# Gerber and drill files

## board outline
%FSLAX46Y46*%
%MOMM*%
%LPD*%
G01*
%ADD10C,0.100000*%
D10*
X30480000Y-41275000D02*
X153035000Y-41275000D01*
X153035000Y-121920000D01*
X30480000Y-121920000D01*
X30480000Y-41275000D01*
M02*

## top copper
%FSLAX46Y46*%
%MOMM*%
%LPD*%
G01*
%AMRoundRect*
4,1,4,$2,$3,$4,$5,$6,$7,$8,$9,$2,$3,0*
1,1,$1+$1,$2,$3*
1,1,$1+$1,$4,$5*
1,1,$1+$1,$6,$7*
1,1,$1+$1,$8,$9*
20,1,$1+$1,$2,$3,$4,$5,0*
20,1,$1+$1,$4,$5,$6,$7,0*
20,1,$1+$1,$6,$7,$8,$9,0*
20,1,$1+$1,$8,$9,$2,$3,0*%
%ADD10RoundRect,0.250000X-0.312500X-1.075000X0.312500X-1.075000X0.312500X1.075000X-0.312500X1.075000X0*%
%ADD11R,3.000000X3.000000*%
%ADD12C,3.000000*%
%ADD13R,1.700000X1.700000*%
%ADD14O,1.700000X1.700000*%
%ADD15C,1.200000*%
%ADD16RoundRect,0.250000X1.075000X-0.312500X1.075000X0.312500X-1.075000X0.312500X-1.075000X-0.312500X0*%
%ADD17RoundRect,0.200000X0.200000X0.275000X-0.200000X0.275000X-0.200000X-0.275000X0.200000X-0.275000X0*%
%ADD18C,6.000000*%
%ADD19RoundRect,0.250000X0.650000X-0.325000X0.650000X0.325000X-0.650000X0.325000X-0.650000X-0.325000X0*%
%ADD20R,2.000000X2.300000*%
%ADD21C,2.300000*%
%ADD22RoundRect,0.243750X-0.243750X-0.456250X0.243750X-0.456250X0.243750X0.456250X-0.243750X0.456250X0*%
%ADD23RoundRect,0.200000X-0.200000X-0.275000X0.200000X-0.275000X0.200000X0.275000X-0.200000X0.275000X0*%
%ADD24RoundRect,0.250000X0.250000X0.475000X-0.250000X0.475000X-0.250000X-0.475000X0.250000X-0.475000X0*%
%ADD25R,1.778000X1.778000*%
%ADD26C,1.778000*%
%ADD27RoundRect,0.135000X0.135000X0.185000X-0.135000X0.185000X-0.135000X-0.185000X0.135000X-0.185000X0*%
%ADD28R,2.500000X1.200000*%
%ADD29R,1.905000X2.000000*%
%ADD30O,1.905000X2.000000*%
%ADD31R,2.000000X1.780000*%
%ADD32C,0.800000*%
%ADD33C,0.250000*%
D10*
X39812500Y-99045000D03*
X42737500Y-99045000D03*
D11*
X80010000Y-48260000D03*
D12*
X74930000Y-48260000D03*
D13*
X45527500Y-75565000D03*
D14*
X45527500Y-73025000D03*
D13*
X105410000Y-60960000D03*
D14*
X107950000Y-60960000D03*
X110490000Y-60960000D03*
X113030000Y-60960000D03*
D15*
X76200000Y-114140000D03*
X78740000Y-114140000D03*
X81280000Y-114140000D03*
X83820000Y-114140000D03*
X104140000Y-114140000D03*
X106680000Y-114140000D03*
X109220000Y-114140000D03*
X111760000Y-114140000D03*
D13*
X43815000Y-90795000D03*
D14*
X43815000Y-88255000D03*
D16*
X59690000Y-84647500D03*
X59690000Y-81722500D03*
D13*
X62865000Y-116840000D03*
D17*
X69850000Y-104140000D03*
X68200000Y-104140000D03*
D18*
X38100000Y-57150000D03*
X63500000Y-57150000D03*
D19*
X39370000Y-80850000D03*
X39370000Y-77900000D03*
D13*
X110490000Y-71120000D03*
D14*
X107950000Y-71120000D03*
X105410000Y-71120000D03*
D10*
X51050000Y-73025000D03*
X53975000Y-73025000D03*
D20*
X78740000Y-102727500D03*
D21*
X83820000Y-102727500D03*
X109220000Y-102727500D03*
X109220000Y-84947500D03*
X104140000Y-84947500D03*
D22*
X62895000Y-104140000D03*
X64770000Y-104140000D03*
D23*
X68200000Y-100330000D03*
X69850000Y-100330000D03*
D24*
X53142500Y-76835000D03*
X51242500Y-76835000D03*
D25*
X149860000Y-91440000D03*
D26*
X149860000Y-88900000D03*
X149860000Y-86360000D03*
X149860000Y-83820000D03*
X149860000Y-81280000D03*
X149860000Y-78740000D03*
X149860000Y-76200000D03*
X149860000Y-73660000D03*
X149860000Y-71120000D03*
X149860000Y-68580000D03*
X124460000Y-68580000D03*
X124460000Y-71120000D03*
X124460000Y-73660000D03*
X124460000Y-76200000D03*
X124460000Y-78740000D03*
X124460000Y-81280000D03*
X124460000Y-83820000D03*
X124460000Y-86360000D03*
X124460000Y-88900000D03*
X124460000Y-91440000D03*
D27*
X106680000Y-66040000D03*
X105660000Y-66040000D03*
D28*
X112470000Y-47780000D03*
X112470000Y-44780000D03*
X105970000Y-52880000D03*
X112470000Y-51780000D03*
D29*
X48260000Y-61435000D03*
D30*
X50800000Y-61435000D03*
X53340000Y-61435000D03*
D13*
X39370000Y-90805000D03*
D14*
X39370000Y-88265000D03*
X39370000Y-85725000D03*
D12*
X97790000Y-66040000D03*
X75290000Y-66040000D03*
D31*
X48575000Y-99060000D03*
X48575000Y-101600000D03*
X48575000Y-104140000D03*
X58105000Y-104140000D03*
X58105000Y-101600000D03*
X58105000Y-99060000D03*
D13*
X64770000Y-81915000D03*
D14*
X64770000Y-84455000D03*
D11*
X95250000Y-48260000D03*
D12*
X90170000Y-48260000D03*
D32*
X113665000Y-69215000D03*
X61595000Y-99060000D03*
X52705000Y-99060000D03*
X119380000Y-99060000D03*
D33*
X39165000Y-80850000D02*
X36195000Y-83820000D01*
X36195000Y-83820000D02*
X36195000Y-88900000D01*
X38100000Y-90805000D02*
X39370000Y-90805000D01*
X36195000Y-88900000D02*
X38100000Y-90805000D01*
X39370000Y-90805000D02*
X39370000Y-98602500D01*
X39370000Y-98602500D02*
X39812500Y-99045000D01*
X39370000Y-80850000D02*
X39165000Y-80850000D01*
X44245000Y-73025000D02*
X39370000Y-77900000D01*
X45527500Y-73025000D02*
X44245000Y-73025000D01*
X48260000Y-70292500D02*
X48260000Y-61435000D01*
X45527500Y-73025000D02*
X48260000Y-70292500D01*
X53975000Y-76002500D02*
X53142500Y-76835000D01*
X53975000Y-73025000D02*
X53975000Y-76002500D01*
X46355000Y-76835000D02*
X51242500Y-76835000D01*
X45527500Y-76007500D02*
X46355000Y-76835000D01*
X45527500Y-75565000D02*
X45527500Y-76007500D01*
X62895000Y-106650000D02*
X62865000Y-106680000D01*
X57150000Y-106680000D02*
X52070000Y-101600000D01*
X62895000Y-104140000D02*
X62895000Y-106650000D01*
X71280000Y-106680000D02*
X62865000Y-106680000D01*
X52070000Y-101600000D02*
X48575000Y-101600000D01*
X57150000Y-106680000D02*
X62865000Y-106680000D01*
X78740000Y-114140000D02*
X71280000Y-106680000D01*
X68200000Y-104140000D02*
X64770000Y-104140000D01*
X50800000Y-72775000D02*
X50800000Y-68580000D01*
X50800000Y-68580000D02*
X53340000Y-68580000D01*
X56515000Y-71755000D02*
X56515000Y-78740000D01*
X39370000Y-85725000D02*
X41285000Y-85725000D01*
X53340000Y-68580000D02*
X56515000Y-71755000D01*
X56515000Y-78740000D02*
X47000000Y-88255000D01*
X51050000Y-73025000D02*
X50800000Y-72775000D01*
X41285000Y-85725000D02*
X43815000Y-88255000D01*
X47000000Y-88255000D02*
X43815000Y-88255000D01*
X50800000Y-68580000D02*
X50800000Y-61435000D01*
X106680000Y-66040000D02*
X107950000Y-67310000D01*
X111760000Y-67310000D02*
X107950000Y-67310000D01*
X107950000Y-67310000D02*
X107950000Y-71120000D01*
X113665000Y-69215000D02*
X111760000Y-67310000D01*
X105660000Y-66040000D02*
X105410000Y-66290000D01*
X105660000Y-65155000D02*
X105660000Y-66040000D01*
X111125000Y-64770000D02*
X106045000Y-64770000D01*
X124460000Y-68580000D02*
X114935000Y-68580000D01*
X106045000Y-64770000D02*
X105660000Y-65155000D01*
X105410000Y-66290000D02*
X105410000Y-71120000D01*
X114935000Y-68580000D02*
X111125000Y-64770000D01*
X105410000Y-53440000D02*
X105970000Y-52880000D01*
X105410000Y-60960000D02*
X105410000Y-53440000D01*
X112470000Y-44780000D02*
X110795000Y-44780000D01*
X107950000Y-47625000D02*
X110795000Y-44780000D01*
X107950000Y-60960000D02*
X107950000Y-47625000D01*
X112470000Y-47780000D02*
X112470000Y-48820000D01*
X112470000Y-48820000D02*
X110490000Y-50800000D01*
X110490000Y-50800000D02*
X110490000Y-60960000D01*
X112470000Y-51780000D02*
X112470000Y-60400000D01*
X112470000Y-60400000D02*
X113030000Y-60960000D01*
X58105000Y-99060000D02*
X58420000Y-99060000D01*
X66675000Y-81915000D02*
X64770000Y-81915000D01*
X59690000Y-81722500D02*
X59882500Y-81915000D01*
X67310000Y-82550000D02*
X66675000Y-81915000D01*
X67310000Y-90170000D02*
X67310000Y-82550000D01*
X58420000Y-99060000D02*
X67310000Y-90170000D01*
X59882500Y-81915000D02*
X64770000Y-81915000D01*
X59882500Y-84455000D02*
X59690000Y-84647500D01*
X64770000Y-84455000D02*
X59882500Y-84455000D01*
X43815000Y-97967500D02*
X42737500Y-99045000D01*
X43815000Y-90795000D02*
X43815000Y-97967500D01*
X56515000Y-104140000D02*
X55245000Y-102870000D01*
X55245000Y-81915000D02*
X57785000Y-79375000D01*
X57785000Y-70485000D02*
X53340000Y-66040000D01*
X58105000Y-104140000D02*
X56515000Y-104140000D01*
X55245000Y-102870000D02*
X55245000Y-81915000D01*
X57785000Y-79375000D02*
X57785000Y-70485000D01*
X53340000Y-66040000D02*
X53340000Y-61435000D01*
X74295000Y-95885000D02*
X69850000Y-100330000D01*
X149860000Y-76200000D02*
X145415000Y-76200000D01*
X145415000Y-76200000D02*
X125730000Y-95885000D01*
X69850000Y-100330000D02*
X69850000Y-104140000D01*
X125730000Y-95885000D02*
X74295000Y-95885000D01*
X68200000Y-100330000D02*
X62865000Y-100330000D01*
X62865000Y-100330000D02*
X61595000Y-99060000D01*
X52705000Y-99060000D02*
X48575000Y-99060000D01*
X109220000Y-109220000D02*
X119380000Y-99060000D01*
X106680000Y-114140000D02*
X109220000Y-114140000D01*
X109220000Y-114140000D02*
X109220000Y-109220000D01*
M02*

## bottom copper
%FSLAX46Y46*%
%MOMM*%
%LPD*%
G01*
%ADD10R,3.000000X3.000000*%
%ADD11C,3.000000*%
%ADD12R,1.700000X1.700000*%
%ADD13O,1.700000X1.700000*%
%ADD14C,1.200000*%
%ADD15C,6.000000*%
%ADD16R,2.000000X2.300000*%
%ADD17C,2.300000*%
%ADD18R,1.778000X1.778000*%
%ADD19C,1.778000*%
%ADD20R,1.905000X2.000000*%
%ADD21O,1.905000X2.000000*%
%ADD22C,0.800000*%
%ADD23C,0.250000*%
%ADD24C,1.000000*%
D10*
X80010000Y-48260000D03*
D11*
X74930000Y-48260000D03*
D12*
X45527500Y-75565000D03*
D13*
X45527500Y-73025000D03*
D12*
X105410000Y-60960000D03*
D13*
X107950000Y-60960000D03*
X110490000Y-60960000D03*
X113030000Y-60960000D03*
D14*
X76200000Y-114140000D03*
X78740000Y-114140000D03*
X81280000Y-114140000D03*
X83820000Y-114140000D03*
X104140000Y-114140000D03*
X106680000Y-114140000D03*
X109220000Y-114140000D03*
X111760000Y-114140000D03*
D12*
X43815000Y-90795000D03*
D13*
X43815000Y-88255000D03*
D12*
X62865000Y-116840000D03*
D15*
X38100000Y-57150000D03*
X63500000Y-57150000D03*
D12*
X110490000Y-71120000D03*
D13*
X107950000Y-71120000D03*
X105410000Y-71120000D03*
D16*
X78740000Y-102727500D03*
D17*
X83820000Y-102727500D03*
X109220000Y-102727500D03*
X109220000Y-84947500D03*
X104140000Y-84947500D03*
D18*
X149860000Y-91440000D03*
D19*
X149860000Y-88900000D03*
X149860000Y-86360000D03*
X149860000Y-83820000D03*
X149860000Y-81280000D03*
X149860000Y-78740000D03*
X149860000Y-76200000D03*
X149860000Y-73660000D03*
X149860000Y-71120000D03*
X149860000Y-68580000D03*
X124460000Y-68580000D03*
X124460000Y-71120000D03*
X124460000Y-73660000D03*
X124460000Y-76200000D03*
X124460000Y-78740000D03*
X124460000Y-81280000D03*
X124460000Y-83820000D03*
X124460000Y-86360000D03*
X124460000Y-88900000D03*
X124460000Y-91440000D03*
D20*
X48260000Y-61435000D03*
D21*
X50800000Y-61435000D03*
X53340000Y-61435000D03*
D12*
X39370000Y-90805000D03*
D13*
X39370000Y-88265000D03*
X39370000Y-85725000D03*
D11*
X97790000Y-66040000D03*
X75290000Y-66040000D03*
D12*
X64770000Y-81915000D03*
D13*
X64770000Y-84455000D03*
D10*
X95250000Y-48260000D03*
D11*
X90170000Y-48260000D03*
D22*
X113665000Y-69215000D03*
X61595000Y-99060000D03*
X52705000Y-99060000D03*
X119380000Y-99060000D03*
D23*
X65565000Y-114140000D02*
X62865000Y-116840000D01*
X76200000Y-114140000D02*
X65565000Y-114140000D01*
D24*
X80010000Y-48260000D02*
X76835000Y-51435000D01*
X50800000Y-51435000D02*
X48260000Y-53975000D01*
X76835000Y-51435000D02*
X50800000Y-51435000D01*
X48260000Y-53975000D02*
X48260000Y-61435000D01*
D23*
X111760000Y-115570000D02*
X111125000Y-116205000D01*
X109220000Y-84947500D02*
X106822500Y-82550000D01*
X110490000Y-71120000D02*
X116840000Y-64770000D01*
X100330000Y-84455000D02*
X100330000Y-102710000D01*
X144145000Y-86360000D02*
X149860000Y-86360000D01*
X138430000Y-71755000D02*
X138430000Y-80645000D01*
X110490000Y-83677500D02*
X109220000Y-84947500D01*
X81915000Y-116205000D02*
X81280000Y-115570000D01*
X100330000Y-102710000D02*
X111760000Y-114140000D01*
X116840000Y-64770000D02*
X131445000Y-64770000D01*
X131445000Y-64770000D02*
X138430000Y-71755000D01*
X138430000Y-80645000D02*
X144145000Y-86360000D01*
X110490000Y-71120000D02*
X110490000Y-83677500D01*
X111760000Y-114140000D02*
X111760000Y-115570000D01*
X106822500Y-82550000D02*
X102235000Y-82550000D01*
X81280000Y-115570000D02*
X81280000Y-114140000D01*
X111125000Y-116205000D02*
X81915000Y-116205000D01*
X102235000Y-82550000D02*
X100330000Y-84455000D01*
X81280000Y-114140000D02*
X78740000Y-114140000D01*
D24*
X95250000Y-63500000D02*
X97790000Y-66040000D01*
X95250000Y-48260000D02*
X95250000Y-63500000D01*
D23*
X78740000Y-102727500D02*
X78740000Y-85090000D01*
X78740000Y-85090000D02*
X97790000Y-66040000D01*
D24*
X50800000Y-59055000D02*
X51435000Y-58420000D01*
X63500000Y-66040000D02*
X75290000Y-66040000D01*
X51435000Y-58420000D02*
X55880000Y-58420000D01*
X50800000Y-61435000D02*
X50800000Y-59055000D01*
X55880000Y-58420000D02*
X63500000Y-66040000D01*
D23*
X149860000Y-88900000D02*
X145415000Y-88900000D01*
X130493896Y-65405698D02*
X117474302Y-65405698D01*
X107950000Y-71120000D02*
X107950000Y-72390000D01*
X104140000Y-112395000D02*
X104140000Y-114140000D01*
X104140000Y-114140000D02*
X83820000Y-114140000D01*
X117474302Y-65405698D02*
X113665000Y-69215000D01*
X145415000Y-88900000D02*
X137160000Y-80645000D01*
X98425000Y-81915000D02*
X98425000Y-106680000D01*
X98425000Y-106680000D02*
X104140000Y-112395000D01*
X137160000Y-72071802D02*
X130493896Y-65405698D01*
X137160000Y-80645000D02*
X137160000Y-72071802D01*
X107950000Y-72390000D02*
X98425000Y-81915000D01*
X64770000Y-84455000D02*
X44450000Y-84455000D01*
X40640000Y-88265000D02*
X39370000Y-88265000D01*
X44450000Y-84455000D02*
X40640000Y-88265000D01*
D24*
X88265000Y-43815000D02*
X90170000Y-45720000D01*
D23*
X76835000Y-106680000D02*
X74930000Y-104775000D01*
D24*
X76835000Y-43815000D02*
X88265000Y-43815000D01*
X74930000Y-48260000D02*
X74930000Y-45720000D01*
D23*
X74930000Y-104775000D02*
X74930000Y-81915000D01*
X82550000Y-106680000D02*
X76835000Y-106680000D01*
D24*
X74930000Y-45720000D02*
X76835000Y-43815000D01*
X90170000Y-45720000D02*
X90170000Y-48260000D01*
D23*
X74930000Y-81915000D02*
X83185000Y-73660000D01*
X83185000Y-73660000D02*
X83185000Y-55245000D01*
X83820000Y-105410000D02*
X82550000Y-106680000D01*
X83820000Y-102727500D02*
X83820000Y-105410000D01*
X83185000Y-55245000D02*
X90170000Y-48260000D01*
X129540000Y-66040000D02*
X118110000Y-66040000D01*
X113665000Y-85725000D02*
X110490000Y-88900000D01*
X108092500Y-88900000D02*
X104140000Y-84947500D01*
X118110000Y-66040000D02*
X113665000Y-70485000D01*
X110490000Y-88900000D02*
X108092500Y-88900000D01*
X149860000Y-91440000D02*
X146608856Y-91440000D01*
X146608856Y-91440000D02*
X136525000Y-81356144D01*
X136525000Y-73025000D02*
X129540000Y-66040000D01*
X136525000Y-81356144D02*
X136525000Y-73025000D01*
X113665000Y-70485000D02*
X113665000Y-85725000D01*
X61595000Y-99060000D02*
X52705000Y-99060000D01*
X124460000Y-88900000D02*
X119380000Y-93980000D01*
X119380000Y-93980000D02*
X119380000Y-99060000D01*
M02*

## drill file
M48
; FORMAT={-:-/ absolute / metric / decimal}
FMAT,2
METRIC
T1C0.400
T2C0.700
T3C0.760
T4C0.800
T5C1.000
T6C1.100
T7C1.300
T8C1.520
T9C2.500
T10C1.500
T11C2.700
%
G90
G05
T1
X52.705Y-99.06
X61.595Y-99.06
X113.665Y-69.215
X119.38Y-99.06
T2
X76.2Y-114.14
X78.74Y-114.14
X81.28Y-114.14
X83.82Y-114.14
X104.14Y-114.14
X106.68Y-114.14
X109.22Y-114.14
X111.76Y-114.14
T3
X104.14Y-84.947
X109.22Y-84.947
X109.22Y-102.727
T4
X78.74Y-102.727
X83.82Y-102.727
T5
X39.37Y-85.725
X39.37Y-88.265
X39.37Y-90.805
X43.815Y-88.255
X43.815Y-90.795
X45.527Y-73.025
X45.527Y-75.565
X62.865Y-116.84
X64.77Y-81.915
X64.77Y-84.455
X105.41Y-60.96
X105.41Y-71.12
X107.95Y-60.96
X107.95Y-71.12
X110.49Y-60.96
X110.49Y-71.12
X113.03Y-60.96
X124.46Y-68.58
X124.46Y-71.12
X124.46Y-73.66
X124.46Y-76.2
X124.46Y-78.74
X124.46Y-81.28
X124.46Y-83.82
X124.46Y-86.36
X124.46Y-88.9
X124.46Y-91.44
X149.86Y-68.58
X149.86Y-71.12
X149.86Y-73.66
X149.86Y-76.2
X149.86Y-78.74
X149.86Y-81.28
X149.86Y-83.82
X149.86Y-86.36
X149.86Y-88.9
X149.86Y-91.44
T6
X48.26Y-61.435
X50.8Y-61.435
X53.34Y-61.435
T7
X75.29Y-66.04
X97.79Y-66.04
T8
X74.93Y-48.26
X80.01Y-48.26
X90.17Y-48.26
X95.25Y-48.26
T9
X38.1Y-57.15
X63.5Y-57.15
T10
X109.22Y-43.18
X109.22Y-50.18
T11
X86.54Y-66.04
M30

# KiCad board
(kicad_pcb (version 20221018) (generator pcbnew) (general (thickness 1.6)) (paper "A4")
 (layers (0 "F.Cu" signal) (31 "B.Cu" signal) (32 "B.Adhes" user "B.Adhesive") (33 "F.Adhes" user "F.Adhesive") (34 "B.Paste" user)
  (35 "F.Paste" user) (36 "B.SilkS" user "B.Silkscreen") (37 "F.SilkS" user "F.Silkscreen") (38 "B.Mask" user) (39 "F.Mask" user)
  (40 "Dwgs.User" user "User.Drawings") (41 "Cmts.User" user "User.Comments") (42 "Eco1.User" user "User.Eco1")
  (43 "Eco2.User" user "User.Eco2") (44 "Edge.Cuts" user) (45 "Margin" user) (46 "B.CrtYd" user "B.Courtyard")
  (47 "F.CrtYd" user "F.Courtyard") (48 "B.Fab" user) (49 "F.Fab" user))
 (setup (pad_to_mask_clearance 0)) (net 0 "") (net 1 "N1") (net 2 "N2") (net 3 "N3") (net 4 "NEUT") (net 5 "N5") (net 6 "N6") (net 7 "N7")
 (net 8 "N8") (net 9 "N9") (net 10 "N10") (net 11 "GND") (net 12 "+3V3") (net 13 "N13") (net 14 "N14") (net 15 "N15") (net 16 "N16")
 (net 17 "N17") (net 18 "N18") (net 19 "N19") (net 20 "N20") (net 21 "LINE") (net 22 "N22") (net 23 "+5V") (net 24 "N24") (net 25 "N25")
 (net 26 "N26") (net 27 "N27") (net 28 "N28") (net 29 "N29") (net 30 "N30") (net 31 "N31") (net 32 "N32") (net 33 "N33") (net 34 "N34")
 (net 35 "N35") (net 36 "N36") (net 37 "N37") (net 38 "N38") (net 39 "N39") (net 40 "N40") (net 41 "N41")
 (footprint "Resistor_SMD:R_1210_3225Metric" (layer "F.Cu") (at 41.275 99.045)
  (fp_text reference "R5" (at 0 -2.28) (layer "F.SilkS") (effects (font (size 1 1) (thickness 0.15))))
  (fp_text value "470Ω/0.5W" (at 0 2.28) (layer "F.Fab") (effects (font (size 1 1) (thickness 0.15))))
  (pad "1" smd roundrect (at -1.4625 0) (size 1.125 2.65) (layers "F.Cu" "F.Paste" "F.Mask") (roundrect_rratio 0.222222) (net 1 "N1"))
  (pad "2" smd roundrect (at 1.4625 0) (size 1.125 2.65) (layers "F.Cu" "F.Paste" "F.Mask") (roundrect_rratio 0.222222) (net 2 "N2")))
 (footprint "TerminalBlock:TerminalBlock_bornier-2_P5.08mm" (layer "F.Cu") (at 80.01 48.26 180)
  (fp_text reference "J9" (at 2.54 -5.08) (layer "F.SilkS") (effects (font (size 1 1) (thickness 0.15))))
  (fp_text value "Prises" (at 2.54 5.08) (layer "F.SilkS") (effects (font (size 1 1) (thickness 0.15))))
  (pad "1" thru_hole rect (at 0 0 180) (size 3 3) (drill 1.52) (layers "*.Cu" "*.Mask") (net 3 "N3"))
  (pad "2" thru_hole circle (at 5.08 0 180) (size 3 3) (drill 1.52) (layers "*.Cu" "*.Mask") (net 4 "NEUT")))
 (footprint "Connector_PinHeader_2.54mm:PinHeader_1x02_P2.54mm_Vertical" (layer "F.Cu") (at 45.5275 75.565 180)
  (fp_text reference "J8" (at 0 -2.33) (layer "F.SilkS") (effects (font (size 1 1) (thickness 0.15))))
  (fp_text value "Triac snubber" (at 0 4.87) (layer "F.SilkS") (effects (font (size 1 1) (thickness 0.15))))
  (pad "1" thru_hole rect (at 0 0 180) (size 1.7 1.7) (drill 1) (layers "*.Cu" "*.Mask") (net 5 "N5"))
  (pad "2" thru_hole oval (at 0 2.54 180) (size 1.7 1.7) (drill 1) (layers "*.Cu" "*.Mask") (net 3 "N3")))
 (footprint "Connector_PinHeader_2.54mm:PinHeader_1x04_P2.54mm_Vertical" (layer "F.Cu") (at 105.41 60.96 90)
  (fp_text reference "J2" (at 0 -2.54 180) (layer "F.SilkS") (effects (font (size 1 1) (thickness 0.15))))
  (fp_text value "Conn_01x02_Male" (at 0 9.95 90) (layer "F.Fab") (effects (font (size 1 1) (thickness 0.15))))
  (pad "1" thru_hole rect (at 0 0 90) (size 1.7 1.7) (drill 1) (layers "*.Cu" "*.Mask") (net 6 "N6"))
  (pad "2" thru_hole oval (at 0 2.54 90) (size 1.7 1.7) (drill 1) (layers "*.Cu" "*.Mask") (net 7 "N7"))
  (pad "3" thru_hole oval (at 0 5.08 90) (size 1.7 1.7) (drill 1) (layers "*.Cu" "*.Mask") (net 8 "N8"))
  (pad "4" thru_hole oval (at 0 7.62 90) (size 1.7 1.7) (drill 1) (layers "*.Cu" "*.Mask") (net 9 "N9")))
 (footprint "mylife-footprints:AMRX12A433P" (layer "F.Cu") (at 93.98 116.84)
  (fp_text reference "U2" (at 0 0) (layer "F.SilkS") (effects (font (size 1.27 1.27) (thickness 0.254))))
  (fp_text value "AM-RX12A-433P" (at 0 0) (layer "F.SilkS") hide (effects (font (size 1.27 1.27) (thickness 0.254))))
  (pad "1" thru_hole circle (at -17.78 -2.7) (size 1.2 1.2) (drill 0.7) (layers "*.Cu" "*.Mask") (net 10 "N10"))
  (pad "2" thru_hole circle (at -15.24 -2.7) (size 1.2 1.2) (drill 0.7) (layers "*.Cu" "*.Mask") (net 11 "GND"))
  (pad "3" thru_hole circle (at -12.7 -2.7) (size 1.2 1.2) (drill 0.7) (layers "*.Cu" "*.Mask") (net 11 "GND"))
  (pad "4" thru_hole circle (at -10.16 -2.7) (size 1.2 1.2) (drill 0.7) (layers "*.Cu" "*.Mask") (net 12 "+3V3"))
  (pad "5" thru_hole circle (at 10.16 -2.7) (size 1.2 1.2) (drill 0.7) (layers "*.Cu" "*.Mask") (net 12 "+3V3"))
  (pad "6" thru_hole circle (at 12.7 -2.7) (size 1.2 1.2) (drill 0.7) (layers "*.Cu" "*.Mask") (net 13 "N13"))
  (pad "7" thru_hole circle (at 15.24 -2.7) (size 1.2 1.2) (drill 0.7) (layers "*.Cu" "*.Mask") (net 13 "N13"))
  (pad "8" thru_hole circle (at 17.78 -2.7) (size 1.2 1.2) (drill 0.7) (layers "*.Cu" "*.Mask") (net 11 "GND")))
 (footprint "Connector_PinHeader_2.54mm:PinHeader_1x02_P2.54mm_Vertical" (layer "F.Cu") (at 43.815 90.795 180)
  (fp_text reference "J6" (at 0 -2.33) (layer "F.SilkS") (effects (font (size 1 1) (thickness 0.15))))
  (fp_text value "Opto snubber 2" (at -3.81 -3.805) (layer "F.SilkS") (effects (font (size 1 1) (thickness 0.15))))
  (pad "1" thru_hole rect (at 0 0 180) (size 1.7 1.7) (drill 1) (layers "*.Cu" "*.Mask") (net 2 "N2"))
  (pad "2" thru_hole oval (at 0 2.54 180) (size 1.7 1.7) (drill 1) (layers "*.Cu" "*.Mask") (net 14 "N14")))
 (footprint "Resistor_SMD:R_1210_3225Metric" (layer "F.Cu") (at 59.69 83.185 90)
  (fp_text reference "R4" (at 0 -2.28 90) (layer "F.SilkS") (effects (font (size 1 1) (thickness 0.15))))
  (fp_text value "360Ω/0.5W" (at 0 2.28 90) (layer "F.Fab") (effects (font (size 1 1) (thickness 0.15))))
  (pad "1" smd roundrect (at -1.4625 0 90) (size 1.125 2.65) (layers "F.Cu" "F.Paste" "F.Mask") (roundrect_rratio 0.222222) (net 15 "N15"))
  (pad "2" smd roundrect (at 1.4625 0 90) (size 1.125 2.65) (layers "F.Cu" "F.Paste" "F.Mask") (roundrect_rratio 0.222222) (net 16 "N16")))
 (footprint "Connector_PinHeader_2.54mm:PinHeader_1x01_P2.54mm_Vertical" (layer "F.Cu") (at 62.865 116.84)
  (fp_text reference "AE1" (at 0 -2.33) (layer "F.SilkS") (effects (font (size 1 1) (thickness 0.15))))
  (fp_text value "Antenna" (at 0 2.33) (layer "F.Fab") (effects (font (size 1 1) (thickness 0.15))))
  (pad "1" thru_hole rect (at 0 0) (size 1.7 1.7) (drill 1) (layers "*.Cu" "*.Mask") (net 10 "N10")))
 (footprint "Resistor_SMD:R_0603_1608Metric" (layer "F.Cu") (at 69.025 104.14 180)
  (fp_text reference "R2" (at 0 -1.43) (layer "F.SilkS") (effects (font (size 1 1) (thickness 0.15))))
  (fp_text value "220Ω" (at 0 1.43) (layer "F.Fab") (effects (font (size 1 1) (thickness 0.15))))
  (pad "1" smd roundrect (at -0.825 0 180) (size 0.8 0.95) (layers "F.Cu" "F.Paste" "F.Mask") (roundrect_rratio 0.25) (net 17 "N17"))
  (pad "2" smd roundrect (at 0.825 0 180) (size 0.8 0.95) (layers "F.Cu" "F.Paste" "F.Mask") (roundrect_rratio 0.25) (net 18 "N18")))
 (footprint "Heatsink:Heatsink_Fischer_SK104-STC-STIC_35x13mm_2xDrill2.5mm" (layer "F.Cu") (at 50.8 57.15)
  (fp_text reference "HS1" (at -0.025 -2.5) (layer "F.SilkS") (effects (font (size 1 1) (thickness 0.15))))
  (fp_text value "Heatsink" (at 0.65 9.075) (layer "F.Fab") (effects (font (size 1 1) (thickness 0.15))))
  (pad "1" thru_hole circle (at -12.7 0 180) (size 6 6) (drill 2.5) (layers "*.Cu" "*.Mask"))
  (pad "1" thru_hole circle (at 12.7 0) (size 6 6) (drill 2.5) (layers "*.Cu" "*.Mask")))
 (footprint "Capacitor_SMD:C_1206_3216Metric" (layer "F.Cu") (at 39.37 79.375 90)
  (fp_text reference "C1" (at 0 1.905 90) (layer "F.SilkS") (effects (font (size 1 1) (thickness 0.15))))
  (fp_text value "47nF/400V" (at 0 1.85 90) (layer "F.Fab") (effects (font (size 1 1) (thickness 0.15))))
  (pad "1" smd roundrect (at -1.475 0 90) (size 1.15 1.8) (layers "F.Cu" "F.Paste" "F.Mask") (roundrect_rratio 0.217391) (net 1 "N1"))
  (pad "2" smd roundrect (at 1.475 0 90) (size 1.15 1.8) (layers "F.Cu" "F.Paste" "F.Mask") (roundrect_rratio 0.217391) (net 3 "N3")))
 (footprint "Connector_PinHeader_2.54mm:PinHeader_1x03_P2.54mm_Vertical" (layer "F.Cu") (at 110.49 71.12 -90)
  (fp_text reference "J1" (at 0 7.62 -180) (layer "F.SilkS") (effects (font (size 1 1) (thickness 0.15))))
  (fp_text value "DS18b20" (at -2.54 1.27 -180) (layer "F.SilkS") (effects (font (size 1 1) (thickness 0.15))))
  (pad "1" thru_hole rect (at 0 0 270) (size 1.7 1.7) (drill 1) (layers "*.Cu" "*.Mask") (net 11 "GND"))
  (pad "2" thru_hole oval (at 0 2.54 270) (size 1.7 1.7) (drill 1) (layers "*.Cu" "*.Mask") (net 12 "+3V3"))
  (pad "3" thru_hole oval (at 0 5.08 270) (size 1.7 1.7) (drill 1) (layers "*.Cu" "*.Mask") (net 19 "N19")))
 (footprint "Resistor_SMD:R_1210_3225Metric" (layer "F.Cu") (at 52.5125 73.025)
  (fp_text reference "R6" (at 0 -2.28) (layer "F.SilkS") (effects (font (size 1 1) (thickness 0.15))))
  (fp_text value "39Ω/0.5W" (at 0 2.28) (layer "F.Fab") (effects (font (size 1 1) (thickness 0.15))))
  (pad "1" smd roundrect (at -1.4625 0) (size 1.125 2.65) (layers "F.Cu" "F.Paste" "F.Mask") (roundrect_rratio 0.222222) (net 14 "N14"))
  (pad "2" smd roundrect (at 1.4625 0) (size 1.125 2.65) (layers "F.Cu" "F.Paste" "F.Mask") (roundrect_rratio 0.222222) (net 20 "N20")))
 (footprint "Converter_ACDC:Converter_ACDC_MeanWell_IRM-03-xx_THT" (layer "F.Cu") (at 78.74 102.7275 90)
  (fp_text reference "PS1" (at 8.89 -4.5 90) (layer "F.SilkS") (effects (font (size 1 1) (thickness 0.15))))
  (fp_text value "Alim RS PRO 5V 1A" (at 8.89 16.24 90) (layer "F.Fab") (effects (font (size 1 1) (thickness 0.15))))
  (pad "1" thru_hole rect (at 0 0 90) (size 2.3 2) (drill 0.8) (layers "*.Cu" "*.Mask") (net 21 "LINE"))
  (pad "3" thru_hole circle (at 0 5.08 90) (size 2.3 2.3) (drill 0.8) (layers "*.Cu" "*.Mask") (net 4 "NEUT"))
  (pad "5" thru_hole circle (at 0 30.48 90) (size 2.3 2.3) (drill 0.76) (layers "*.Cu" "*.Mask") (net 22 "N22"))
  (pad "14" thru_hole circle (at 17.78 30.48 90) (size 2.3 2.3) (drill 0.76) (layers "*.Cu" "*.Mask") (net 11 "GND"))
  (pad "16" thru_hole circle (at 17.78 25.4 90) (size 2.3 2.3) (drill 0.76) (layers "*.Cu" "*.Mask") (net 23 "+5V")))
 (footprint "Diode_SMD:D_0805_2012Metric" (layer "F.Cu") (at 63.8325 104.14)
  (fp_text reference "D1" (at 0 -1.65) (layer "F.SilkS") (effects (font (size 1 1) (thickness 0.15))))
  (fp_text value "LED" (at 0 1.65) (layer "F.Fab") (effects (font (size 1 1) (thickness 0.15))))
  (pad "1" smd roundrect (at -0.9375 0) (size 0.975 1.4) (layers "F.Cu" "F.Paste" "F.Mask") (roundrect_rratio 0.25) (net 11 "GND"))
  (pad "2" smd roundrect (at 0.9375 0) (size 0.975 1.4) (layers "F.Cu" "F.Paste" "F.Mask") (roundrect_rratio 0.25) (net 18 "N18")))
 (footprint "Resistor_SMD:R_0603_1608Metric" (layer "F.Cu") (at 69.025 100.33)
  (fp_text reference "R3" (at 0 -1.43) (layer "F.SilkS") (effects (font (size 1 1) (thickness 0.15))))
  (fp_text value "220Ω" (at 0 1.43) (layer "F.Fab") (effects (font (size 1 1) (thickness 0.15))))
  (pad "1" smd roundrect (at -0.825 0) (size 0.8 0.95) (layers "F.Cu" "F.Paste" "F.Mask") (roundrect_rratio 0.25) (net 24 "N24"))
  (pad "2" smd roundrect (at 0.825 0) (size 0.8 0.95) (layers "F.Cu" "F.Paste" "F.Mask") (roundrect_rratio 0.25) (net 17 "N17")))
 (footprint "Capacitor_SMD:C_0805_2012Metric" (layer "F.Cu") (at 52.1925 76.835 180)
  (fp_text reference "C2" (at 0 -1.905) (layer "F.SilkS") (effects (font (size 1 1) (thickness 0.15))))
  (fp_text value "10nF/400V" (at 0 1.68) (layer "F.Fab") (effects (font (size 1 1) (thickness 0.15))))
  (pad "1" smd roundrect (at -0.95 0 180) (size 1 1.45) (layers "F.Cu" "F.Paste" "F.Mask") (roundrect_rratio 0.25) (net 20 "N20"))
  (pad "2" smd roundrect (at 0.95 0 180) (size 1 1.45) (layers "F.Cu" "F.Paste" "F.Mask") (roundrect_rratio 0.25) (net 5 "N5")))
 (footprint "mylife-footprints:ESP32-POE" (layer "F.Cu") (at 137.12 81.41 180)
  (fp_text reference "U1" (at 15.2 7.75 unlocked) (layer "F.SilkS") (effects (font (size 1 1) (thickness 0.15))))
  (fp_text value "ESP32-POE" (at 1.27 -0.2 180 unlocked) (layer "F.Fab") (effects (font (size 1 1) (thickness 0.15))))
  (pad "1" thru_hole rect (at -12.74 -10.03 90) (size 1.778 1.778) (drill 1) (layers "*.Cu" "*.Mask") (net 23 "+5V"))
  (pad "2" thru_hole circle (at -12.74 -7.49 90) (size 1.778 1.778) (drill 1) (layers "*.Cu" "*.Mask") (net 12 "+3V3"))
  (pad "3" thru_hole circle (at -12.74 -4.95 90) (size 1.778 1.778) (drill 1) (layers "*.Cu" "*.Mask") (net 11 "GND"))
  (pad "4" thru_hole circle (at -12.74 -2.41 90) (size 1.778 1.778) (drill 1) (layers "*.Cu" "*.Mask") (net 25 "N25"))
  (pad "5" thru_hole circle (at -12.74 0.13 90) (size 1.778 1.778) (drill 1) (layers "*.Cu" "*.Mask") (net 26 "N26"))
  (pad "6" thru_hole circle (at -12.74 2.67 90) (size 1.778 1.778) (drill 1) (layers "*.Cu" "*.Mask") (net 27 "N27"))
  (pad "7" thru_hole circle (at -12.74 5.21 90) (size 1.778 1.778) (drill 1) (layers "*.Cu" "*.Mask") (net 17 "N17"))
  (pad "8" thru_hole circle (at -12.74 7.75 90) (size 1.778 1.778) (drill 1) (layers "*.Cu" "*.Mask") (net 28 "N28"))
  (pad "9" thru_hole circle (at -12.74 10.29 90) (size 1.778 1.778) (drill 1) (layers "*.Cu" "*.Mask") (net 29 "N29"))
  (pad "10" thru_hole circle (at -12.74 12.83 90) (size 1.778 1.778) (drill 1) (layers "*.Cu" "*.Mask") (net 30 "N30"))
  (pad "11" thru_hole circle (at 12.66 12.83 90) (size 1.778 1.778) (drill 1) (layers "*.Cu" "*.Mask") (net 19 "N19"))
  (pad "12" thru_hole circle (at 12.66 10.29 90) (size 1.778 1.778) (drill 1) (layers "*.Cu" "*.Mask") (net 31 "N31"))
  (pad "13" thru_hole circle (at 12.66 7.75 90) (size 1.778 1.778) (drill 1) (layers "*.Cu" "*.Mask") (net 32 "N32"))
  (pad "14" thru_hole circle (at 12.66 5.21 90) (size 1.778 1.778) (drill 1) (layers "*.Cu" "*.Mask") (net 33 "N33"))
  (pad "15" thru_hole circle (at 12.66 2.67 90) (size 1.778 1.778) (drill 1) (layers "*.Cu" "*.Mask") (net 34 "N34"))
  (pad "16" thru_hole circle (at 12.66 0.13 90) (size 1.778 1.778) (drill 1) (layers "*.Cu" "*.Mask") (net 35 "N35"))
  (pad "17" thru_hole circle (at 12.66 -2.41 90) (size 1.778 1.778) (drill 1) (layers "*.Cu" "*.Mask") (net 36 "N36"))
  (pad "18" thru_hole circle (at 12.66 -4.95 90) (size 1.778 1.778) (drill 1) (layers "*.Cu" "*.Mask") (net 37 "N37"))
  (pad "19" thru_hole circle (at 12.66 -7.49 90) (size 1.778 1.778) (drill 1) (layers "*.Cu" "*.Mask") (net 13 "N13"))
  (pad "20" thru_hole circle (at 12.66 -10.03 90) (size 1.778 1.778) (drill 1) (layers "*.Cu" "*.Mask") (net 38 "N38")))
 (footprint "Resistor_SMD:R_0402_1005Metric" (layer "F.Cu") (at 106.17 66.04 180)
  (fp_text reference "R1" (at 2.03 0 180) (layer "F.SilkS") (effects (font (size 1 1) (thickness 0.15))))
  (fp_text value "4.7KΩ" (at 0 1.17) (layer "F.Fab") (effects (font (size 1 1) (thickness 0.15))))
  (pad "1" smd roundrect (at -0.51 0 180) (size 0.54 0.64) (layers "F.Cu" "F.Paste" "F.Mask") (roundrect_rratio 0.25) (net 12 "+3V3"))
  (pad "2" smd roundrect (at 0.51 0 180) (size 0.54 0.64) (layers "F.Cu" "F.Paste" "F.Mask") (roundrect_rratio 0.25) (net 19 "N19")))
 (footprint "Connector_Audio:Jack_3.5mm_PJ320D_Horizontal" (layer "F.Cu") (at 109.22 47.955 -90)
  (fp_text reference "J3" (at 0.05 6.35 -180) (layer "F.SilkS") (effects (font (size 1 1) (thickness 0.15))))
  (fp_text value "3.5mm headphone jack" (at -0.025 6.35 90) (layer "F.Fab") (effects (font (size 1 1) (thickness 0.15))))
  (pad "" np_thru_hole circle (at -4.775 0 270) (size 1.5 1.5) (drill 1.5) (layers "*.Cu" "*.Mask"))
  (pad "" np_thru_hole circle (at 2.225 0 270) (size 1.5 1.5) (drill 1.5) (layers "*.Cu" "*.Mask"))
  (pad "R1" smd rect (at -0.175 -3.25 270) (size 1.2 2.5) (layers "F.Cu" "F.Paste" "F.Mask") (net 8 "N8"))
  (pad "R2" smd rect (at -3.175 -3.25 270) (size 1.2 2.5) (layers "F.Cu" "F.Paste" "F.Mask") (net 7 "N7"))
  (pad "S" smd rect (at 4.925 3.25 270) (size 1.2 2.5) (layers "F.Cu" "F.Paste" "F.Mask") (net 6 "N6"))
  (pad "T" smd rect (at 3.825 -3.25 270) (size 1.2 2.5) (layers "F.Cu" "F.Paste" "F.Mask") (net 9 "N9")))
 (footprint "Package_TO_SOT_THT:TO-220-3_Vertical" (layer "F.Cu") (at 48.26 61.435)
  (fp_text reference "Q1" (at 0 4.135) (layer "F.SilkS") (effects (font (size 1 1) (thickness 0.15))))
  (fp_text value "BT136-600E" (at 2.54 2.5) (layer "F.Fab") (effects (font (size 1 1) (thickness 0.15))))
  (pad "1" thru_hole rect (at 0 0) (size 1.905 2) (drill 1.1) (layers "*.Cu" "*.Mask") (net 3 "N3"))
  (pad "2" thru_hole oval (at 2.54 0) (size 1.905 2) (drill 1.1) (layers "*.Cu" "*.Mask") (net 14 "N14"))
  (pad "3" thru_hole oval (at 5.08 0) (size 1.905 2) (drill 1.1) (layers "*.Cu" "*.Mask") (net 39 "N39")))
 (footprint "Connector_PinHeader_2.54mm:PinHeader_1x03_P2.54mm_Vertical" (layer "F.Cu") (at 39.37 90.805 180)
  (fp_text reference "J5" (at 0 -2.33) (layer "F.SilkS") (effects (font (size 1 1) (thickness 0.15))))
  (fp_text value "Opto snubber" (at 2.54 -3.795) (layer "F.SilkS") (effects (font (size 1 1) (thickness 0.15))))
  (pad "1" thru_hole rect (at 0 0 180) (size 1.7 1.7) (drill 1) (layers "*.Cu" "*.Mask") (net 1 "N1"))
  (pad "2" thru_hole oval (at 0 2.54 180) (size 1.7 1.7) (drill 1) (layers "*.Cu" "*.Mask") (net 15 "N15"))
  (pad "3" thru_hole oval (at 0 5.08 180) (size 1.7 1.7) (drill 1) (layers "*.Cu" "*.Mask") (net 14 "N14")))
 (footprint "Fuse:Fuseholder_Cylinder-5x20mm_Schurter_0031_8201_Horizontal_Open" (layer "F.Cu") (at 97.79 66.04 180)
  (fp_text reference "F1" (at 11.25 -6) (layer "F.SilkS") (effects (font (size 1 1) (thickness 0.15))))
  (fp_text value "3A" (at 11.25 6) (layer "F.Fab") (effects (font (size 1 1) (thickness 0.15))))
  (pad "" np_thru_hole circle (at 11.25 0 180) (size 2.7 2.7) (drill 2.7) (layers "*.Cu" "*.Mask"))
  (pad "1" thru_hole circle (at 0 0 180) (size 3 3) (drill 1.3) (layers "*.Cu" "*.Mask") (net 21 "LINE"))
  (pad "2" thru_hole circle (at 22.5 0 180) (size 3 3) (drill 1.3) (layers "*.Cu" "*.Mask") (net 14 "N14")))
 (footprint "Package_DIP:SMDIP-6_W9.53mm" (layer "F.Cu") (at 53.34 101.6)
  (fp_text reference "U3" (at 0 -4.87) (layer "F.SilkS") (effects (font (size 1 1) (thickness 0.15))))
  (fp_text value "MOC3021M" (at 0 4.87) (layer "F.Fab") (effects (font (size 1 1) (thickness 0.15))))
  (pad "1" smd rect (at -4.765 -2.54) (size 2 1.78) (layers "F.Cu" "F.Paste" "F.Mask") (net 24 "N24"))
  (pad "2" smd rect (at -4.765 0) (size 2 1.78) (layers "F.Cu" "F.Paste" "F.Mask") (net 11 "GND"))
  (pad "3" smd rect (at -4.765 2.54) (size 2 1.78) (layers "F.Cu" "F.Paste" "F.Mask") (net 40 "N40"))
  (pad "4" smd rect (at 4.765 2.54) (size 2 1.78) (layers "F.Cu" "F.Paste" "F.Mask") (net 39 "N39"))
  (pad "5" smd rect (at 4.765 0) (size 2 1.78) (layers "F.Cu" "F.Paste" "F.Mask") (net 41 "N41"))
  (pad "6" smd rect (at 4.765 -2.54) (size 2 1.78) (layers "F.Cu" "F.Paste" "F.Mask") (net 16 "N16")))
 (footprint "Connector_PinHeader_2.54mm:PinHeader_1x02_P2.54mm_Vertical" (layer "F.Cu") (at 64.77 81.915)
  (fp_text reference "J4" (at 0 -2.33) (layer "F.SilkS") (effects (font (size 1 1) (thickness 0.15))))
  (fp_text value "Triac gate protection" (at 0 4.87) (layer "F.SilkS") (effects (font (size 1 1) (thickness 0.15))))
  (pad "1" thru_hole rect (at 0 0) (size 1.7 1.7) (drill 1) (layers "*.Cu" "*.Mask") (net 16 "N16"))
  (pad "2" thru_hole oval (at 0 2.54) (size 1.7 1.7) (drill 1) (layers "*.Cu" "*.Mask") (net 15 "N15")))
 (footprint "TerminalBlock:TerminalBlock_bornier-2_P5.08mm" (layer "F.Cu") (at 95.25 48.26 180)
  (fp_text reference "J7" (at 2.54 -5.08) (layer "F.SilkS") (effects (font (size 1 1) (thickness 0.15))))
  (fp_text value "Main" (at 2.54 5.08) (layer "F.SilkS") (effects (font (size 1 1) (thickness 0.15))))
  (pad "1" thru_hole rect (at 0 0 180) (size 3 3) (drill 1.52) (layers "*.Cu" "*.Mask") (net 21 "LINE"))
  (pad "2" thru_hole circle (at 5.08 0 180) (size 3 3) (drill 1.52) (layers "*.Cu" "*.Mask") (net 4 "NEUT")))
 (gr_rect (start 30.48 41.275) (end 153.035 121.92) (stroke (width 0.1) (type default)) (fill none) (layer "Edge.Cuts"))
 (segment (start 65.565 114.14) (end 62.865 116.84) (width 0.25) (layer "B.Cu") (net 10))
 (segment (start 76.2 114.14) (end 65.565 114.14) (width 0.25) (layer "B.Cu") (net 10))
 (segment (start 39.165 80.85) (end 36.195 83.82) (width 0.25) (layer "F.Cu") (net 1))
 (segment (start 36.195 83.82) (end 36.195 88.9) (width 0.25) (layer "F.Cu") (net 1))
 (segment (start 38.1 90.805) (end 39.37 90.805) (width 0.25) (layer "F.Cu") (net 1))
 (segment (start 36.195 88.9) (end 38.1 90.805) (width 0.25) (layer "F.Cu") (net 1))
 (segment (start 39.37 90.805) (end 39.37 98.6025) (width 0.25) (layer "F.Cu") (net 1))
 (segment (start 39.37 98.6025) (end 39.8125 99.045) (width 0.25) (layer "F.Cu") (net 1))
 (segment (start 39.37 80.85) (end 39.165 80.85) (width 0.25) (layer "F.Cu") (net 1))
 (segment (start 44.245 73.025) (end 39.37 77.9) (width 0.25) (layer "F.Cu") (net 3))
 (segment (start 45.5275 73.025) (end 44.245 73.025) (width 0.25) (layer "F.Cu") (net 3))
 (segment (start 48.26 70.2925) (end 48.26 61.435) (width 0.25) (layer "F.Cu") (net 3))
 (segment (start 45.5275 73.025) (end 48.26 70.2925) (width 0.25) (layer "F.Cu") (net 3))
 (segment (start 80.01 48.26) (end 76.835 51.435) (width 1) (layer "B.Cu") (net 3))
 (segment (start 50.8 51.435) (end 48.26 53.975) (width 1) (layer "B.Cu") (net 3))
 (segment (start 76.835 51.435) (end 50.8 51.435) (width 1) (layer "B.Cu") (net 3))
 (segment (start 48.26 53.975) (end 48.26 61.435) (width 1) (layer "B.Cu") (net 3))
 (segment (start 53.975 76.0025) (end 53.1425 76.835) (width 0.25) (layer "F.Cu") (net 20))
 (segment (start 53.975 73.025) (end 53.975 76.0025) (width 0.25) (layer "F.Cu") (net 20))
 (segment (start 46.355 76.835) (end 51.2425 76.835) (width 0.25) (layer "F.Cu") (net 5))
 (segment (start 45.5275 76.0075) (end 46.355 76.835) (width 0.25) (layer "F.Cu") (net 5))
 (segment (start 45.5275 75.565) (end 45.5275 76.0075) (width 0.25) (layer "F.Cu") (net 5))
 (segment (start 62.895 106.65) (end 62.865 106.68) (width 0.25) (layer "F.Cu") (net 11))
 (segment (start 57.15 106.68) (end 52.07 101.6) (width 0.25) (layer "F.Cu") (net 11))
 (segment (start 62.895 104.14) (end 62.895 106.65) (width 0.25) (layer "F.Cu") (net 11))
 (segment (start 71.28 106.68) (end 62.865 106.68) (width 0.25) (layer "F.Cu") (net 11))
 (segment (start 52.07 101.6) (end 48.575 101.6) (width 0.25) (layer "F.Cu") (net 11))
 (segment (start 57.15 106.68) (end 62.865 106.68) (width 0.25) (layer "F.Cu") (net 11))
 (segment (start 78.74 114.14) (end 71.28 106.68) (width 0.25) (layer "F.Cu") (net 11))
 (segment (start 111.76 115.57) (end 111.125 116.205) (width 0.25) (layer "B.Cu") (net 11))
 (segment (start 109.22 84.9475) (end 106.8225 82.55) (width 0.25) (layer "B.Cu") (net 11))
 (segment (start 110.49 71.12) (end 116.84 64.77) (width 0.25) (layer "B.Cu") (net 11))
 (segment (start 100.33 84.455) (end 100.33 102.71) (width 0.25) (layer "B.Cu") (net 11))
 (segment (start 144.145 86.36) (end 149.86 86.36) (width 0.25) (layer "B.Cu") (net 11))
 (segment (start 138.43 71.755) (end 138.43 80.645) (width 0.25) (layer "B.Cu") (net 11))
 (segment (start 110.49 83.6775) (end 109.22 84.9475) (width 0.25) (layer "B.Cu") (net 11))
 (segment (start 81.915 116.205) (end 81.28 115.57) (width 0.25) (layer "B.Cu") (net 11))
 (segment (start 100.33 102.71) (end 111.76 114.14) (width 0.25) (layer "B.Cu") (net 11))
 (segment (start 116.84 64.77) (end 131.445 64.77) (width 0.25) (layer "B.Cu") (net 11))
 (segment (start 131.445 64.77) (end 138.43 71.755) (width 0.25) (layer "B.Cu") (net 11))
 (segment (start 138.43 80.645) (end 144.145 86.36) (width 0.25) (layer "B.Cu") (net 11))
 (segment (start 110.49 71.12) (end 110.49 83.6775) (width 0.25) (layer "B.Cu") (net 11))
 (segment (start 111.76 114.14) (end 111.76 115.57) (width 0.25) (layer "B.Cu") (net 11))
 (segment (start 106.8225 82.55) (end 102.235 82.55) (width 0.25) (layer "B.Cu") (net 11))
 (segment (start 81.28 115.57) (end 81.28 114.14) (width 0.25) (layer "B.Cu") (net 11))
 (segment (start 111.125 116.205) (end 81.915 116.205) (width 0.25) (layer "B.Cu") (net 11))
 (segment (start 102.235 82.55) (end 100.33 84.455) (width 0.25) (layer "B.Cu") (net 11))
 (segment (start 81.28 114.14) (end 78.74 114.14) (width 0.25) (layer "B.Cu") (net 11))
 (segment (start 68.2 104.14) (end 64.77 104.14) (width 0.25) (layer "F.Cu") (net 18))
 (segment (start 95.25 63.5) (end 97.79 66.04) (width 1) (layer "B.Cu") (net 21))
 (segment (start 95.25 48.26) (end 95.25 63.5) (width 1) (layer "B.Cu") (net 21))
 (segment (start 78.74 102.7275) (end 78.74 85.09) (width 0.25) (layer "B.Cu") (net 21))
 (segment (start 78.74 85.09) (end 97.79 66.04) (width 0.25) (layer "B.Cu") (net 21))
 (segment (start 50.8 72.775) (end 50.8 68.58) (width 0.25) (layer "F.Cu") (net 14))
 (segment (start 50.8 68.58) (end 53.34 68.58) (width 0.25) (layer "F.Cu") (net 14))
 (segment (start 56.515 71.755) (end 56.515 78.74) (width 0.25) (layer "F.Cu") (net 14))
 (segment (start 39.37 85.725) (end 41.285 85.725) (width 0.25) (layer "F.Cu") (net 14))
 (segment (start 53.34 68.58) (end 56.515 71.755) (width 0.25) (layer "F.Cu") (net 14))
 (segment (start 56.515 78.74) (end 47 88.255) (width 0.25) (layer "F.Cu") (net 14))
 (segment (start 51.05 73.025) (end 50.8 72.775) (width 0.25) (layer "F.Cu") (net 14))
 (segment (start 41.285 85.725) (end 43.815 88.255) (width 0.25) (layer "F.Cu") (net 14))
 (segment (start 47 88.255) (end 43.815 88.255) (width 0.25) (layer "F.Cu") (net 14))
 (segment (start 50.8 68.58) (end 50.8 61.435) (width 0.25) (layer "F.Cu") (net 14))
 (segment (start 50.8 59.055) (end 51.435 58.42) (width 1) (layer "B.Cu") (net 14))
 (segment (start 63.5 66.04) (end 75.29 66.04) (width 1) (layer "B.Cu") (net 14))
 (segment (start 51.435 58.42) (end 55.88 58.42) (width 1) (layer "B.Cu") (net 14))
 (segment (start 50.8 61.435) (end 50.8 59.055) (width 1) (layer "B.Cu") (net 14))
 (segment (start 55.88 58.42) (end 63.5 66.04) (width 1) (layer "B.Cu") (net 14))
 (segment (start 106.68 66.04) (end 107.95 67.31) (width 0.25) (layer "F.Cu") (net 12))
 (segment (start 111.76 67.31) (end 107.95 67.31) (width 0.25) (layer "F.Cu") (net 12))
 (segment (start 107.95 67.31) (end 107.95 71.12) (width 0.25) (layer "F.Cu") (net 12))
 (segment (start 113.665 69.215) (end 111.76 67.31) (width 0.25) (layer "F.Cu") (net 12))
 (via (at 113.665 69.215) (size 0.8) (drill 0.4) (layers "F.Cu" "B.Cu") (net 12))
 (segment (start 149.86 88.9) (end 145.415 88.9) (width 0.25) (layer "B.Cu") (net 12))
 (segment (start 130.493896 65.405698) (end 117.474302 65.405698) (width 0.25) (layer "B.Cu") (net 12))
 (segment (start 107.95 71.12) (end 107.95 72.39) (width 0.25) (layer "B.Cu") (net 12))
 (segment (start 104.14 112.395) (end 104.14 114.14) (width 0.25) (layer "B.Cu") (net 12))
 (segment (start 104.14 114.14) (end 83.82 114.14) (width 0.25) (layer "B.Cu") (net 12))
 (segment (start 117.474302 65.405698) (end 113.665 69.215) (width 0.25) (layer "B.Cu") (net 12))
 (segment (start 145.415 88.9) (end 137.16 80.645) (width 0.25) (layer "B.Cu") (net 12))
 (segment (start 98.425 81.915) (end 98.425 106.68) (width 0.25) (layer "B.Cu") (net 12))
 (segment (start 98.425 106.68) (end 104.14 112.395) (width 0.25) (layer "B.Cu") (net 12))
 (segment (start 137.16 72.071802) (end 130.493896 65.405698) (width 0.25) (layer "B.Cu") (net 12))
 (segment (start 137.16 80.645) (end 137.16 72.071802) (width 0.25) (layer "B.Cu") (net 12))
 (segment (start 107.95 72.39) (end 98.425 81.915) (width 0.25) (layer "B.Cu") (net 12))
 (segment (start 105.66 66.04) (end 105.41 66.29) (width 0.25) (layer "F.Cu") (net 19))
 (segment (start 105.66 65.155) (end 105.66 66.04) (width 0.25) (layer "F.Cu") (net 19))
 (segment (start 111.125 64.77) (end 106.045 64.77) (width 0.25) (layer "F.Cu") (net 19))
 (segment (start 124.46 68.58) (end 114.935 68.58) (width 0.25) (layer "F.Cu") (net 19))
 (segment (start 106.045 64.77) (end 105.66 65.155) (width 0.25) (layer "F.Cu") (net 19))
 (segment (start 105.41 66.29) (end 105.41 71.12) (width 0.25) (layer "F.Cu") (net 19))
 (segment (start 114.935 68.58) (end 111.125 64.77) (width 0.25) (layer "F.Cu") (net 19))
 (segment (start 105.41 53.44) (end 105.97 52.88) (width 0.25) (layer "F.Cu") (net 6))
 (segment (start 105.41 60.96) (end 105.41 53.44) (width 0.25) (layer "F.Cu") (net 6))
 (segment (start 112.47 44.78) (end 110.795 44.78) (width 0.25) (layer "F.Cu") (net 7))
 (segment (start 107.95 47.625) (end 110.795 44.78) (width 0.25) (layer "F.Cu") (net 7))
 (segment (start 107.95 60.96) (end 107.95 47.625) (width 0.25) (layer "F.Cu") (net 7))
 (segment (start 112.47 47.78) (end 112.47 48.82) (width 0.25) (layer "F.Cu") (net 8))
 (segment (start 112.47 48.82) (end 110.49 50.8) (width 0.25) (layer "F.Cu") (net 8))
 (segment (start 110.49 50.8) (end 110.49 60.96) (width 0.25) (layer "F.Cu") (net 8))
 (segment (start 112.47 51.78) (end 112.47 60.4) (width 0.25) (layer "F.Cu") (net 9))
 (segment (start 112.47 60.4) (end 113.03 60.96) (width 0.25) (layer "F.Cu") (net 9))
 (segment (start 58.105 99.06) (end 58.42 99.06) (width 0.25) (layer "F.Cu") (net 16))
 (segment (start 66.675 81.915) (end 64.77 81.915) (width 0.25) (layer "F.Cu") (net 16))
 (segment (start 59.69 81.7225) (end 59.8825 81.915) (width 0.25) (layer "F.Cu") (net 16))
 (segment (start 67.31 82.55) (end 66.675 81.915) (width 0.25) (layer "F.Cu") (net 16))
 (segment (start 67.31 90.17) (end 67.31 82.55) (width 0.25) (layer "F.Cu") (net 16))
 (segment (start 58.42 99.06) (end 67.31 90.17) (width 0.25) (layer "F.Cu") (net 16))
 (segment (start 59.8825 81.915) (end 64.77 81.915) (width 0.25) (layer "F.Cu") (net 16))
 (segment (start 59.8825 84.455) (end 59.69 84.6475) (width 0.25) (layer "F.Cu") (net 15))
 (segment (start 64.77 84.455) (end 59.8825 84.455) (width 0.25) (layer "F.Cu") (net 15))
 (segment (start 64.77 84.455) (end 44.45 84.455) (width 0.25) (layer "B.Cu") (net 15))
 (segment (start 40.64 88.265) (end 39.37 88.265) (width 0.25) (layer "B.Cu") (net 15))
 (segment (start 44.45 84.455) (end 40.64 88.265) (width 0.25) (layer "B.Cu") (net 15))
 (segment (start 43.815 97.9675) (end 42.7375 99.045) (width 0.25) (layer "F.Cu") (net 2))
 (segment (start 43.815 90.795) (end 43.815 97.9675) (width 0.25) (layer "F.Cu") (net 2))
 (segment (start 88.265 43.815) (end 90.17 45.72) (width 1) (layer "B.Cu") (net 4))
 (segment (start 76.835 106.68) (end 74.93 104.775) (width 0.25) (layer "B.Cu") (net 4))
 (segment (start 76.835 43.815) (end 88.265 43.815) (width 1) (layer "B.Cu") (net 4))
 (segment (start 74.93 48.26) (end 74.93 45.72) (width 1) (layer "B.Cu") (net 4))
 (segment (start 74.93 104.775) (end 74.93 81.915) (width 0.25) (layer "B.Cu") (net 4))
 (segment (start 82.55 106.68) (end 76.835 106.68) (width 0.25) (layer "B.Cu") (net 4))
 (segment (start 74.93 45.72) (end 76.835 43.815) (width 1) (layer "B.Cu") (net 4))
 (segment (start 90.17 45.72) (end 90.17 48.26) (width 1) (layer "B.Cu") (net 4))
 (segment (start 74.93 81.915) (end 83.185 73.66) (width 0.25) (layer "B.Cu") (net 4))
 (segment (start 83.185 73.66) (end 83.185 55.245) (width 0.25) (layer "B.Cu") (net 4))
 (segment (start 83.82 105.41) (end 82.55 106.68) (width 0.25) (layer "B.Cu") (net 4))
 (segment (start 83.82 102.7275) (end 83.82 105.41) (width 0.25) (layer "B.Cu") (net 4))
 (segment (start 83.185 55.245) (end 90.17 48.26) (width 0.25) (layer "B.Cu") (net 4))
 (segment (start 129.54 66.04) (end 118.11 66.04) (width 0.25) (layer "B.Cu") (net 23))
 (segment (start 113.665 85.725) (end 110.49 88.9) (width 0.25) (layer "B.Cu") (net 23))
 (segment (start 108.0925 88.9) (end 104.14 84.9475) (width 0.25) (layer "B.Cu") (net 23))
 (segment (start 118.11 66.04) (end 113.665 70.485) (width 0.25) (layer "B.Cu") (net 23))
 (segment (start 110.49 88.9) (end 108.0925 88.9) (width 0.25) (layer "B.Cu") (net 23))
 (segment (start 149.86 91.44) (end 146.608856 91.44) (width 0.25) (layer "B.Cu") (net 23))
 (segment (start 146.608856 91.44) (end 136.525 81.356144) (width 0.25) (layer "B.Cu") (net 23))
 (segment (start 136.525 73.025) (end 129.54 66.04) (width 0.25) (layer "B.Cu") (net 23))
 (segment (start 136.525 81.356144) (end 136.525 73.025) (width 0.25) (layer "B.Cu") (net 23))
 (segment (start 113.665 70.485) (end 113.665 85.725) (width 0.25) (layer "B.Cu") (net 23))
 (segment (start 56.515 104.14) (end 55.245 102.87) (width 0.25) (layer "F.Cu") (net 39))
 (segment (start 55.245 81.915) (end 57.785 79.375) (width 0.25) (layer "F.Cu") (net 39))
 (segment (start 57.785 70.485) (end 53.34 66.04) (width 0.25) (layer "F.Cu") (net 39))
 (segment (start 58.105 104.14) (end 56.515 104.14) (width 0.25) (layer "F.Cu") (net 39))
 (segment (start 55.245 102.87) (end 55.245 81.915) (width 0.25) (layer "F.Cu") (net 39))
 (segment (start 57.785 79.375) (end 57.785 70.485) (width 0.25) (layer "F.Cu") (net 39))
 (segment (start 53.34 66.04) (end 53.34 61.435) (width 0.25) (layer "F.Cu") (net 39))
 (segment (start 74.295 95.885) (end 69.85 100.33) (width 0.25) (layer "F.Cu") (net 17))
 (segment (start 149.86 76.2) (end 145.415 76.2) (width 0.25) (layer "F.Cu") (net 17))
 (segment (start 145.415 76.2) (end 125.73 95.885) (width 0.25) (layer "F.Cu") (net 17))
 (segment (start 69.85 100.33) (end 69.85 104.14) (width 0.25) (layer "F.Cu") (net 17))
 (segment (start 125.73 95.885) (end 74.295 95.885) (width 0.25) (layer "F.Cu") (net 17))
 (segment (start 68.2 100.33) (end 62.865 100.33) (width 0.25) (layer "F.Cu") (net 24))
 (segment (start 62.865 100.33) (end 61.595 99.06) (width 0.25) (layer "F.Cu") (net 24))
 (segment (start 52.705 99.06) (end 48.575 99.06) (width 0.25) (layer "F.Cu") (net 24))
 (via (at 61.595 99.06) (size 0.8) (drill 0.4) (layers "F.Cu" "B.Cu") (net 24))
 (via (at 52.705 99.06) (size 0.8) (drill 0.4) (layers "F.Cu" "B.Cu") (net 24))
 (segment (start 61.595 99.06) (end 52.705 99.06) (width 0.25) (layer "B.Cu") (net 24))
 (segment (start 109.22 109.22) (end 119.38 99.06) (width 0.25) (layer "F.Cu") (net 13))
 (segment (start 106.68 114.14) (end 109.22 114.14) (width 0.25) (layer "F.Cu") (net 13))
 (segment (start 109.22 114.14) (end 109.22 109.22) (width 0.25) (layer "F.Cu") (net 13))
 (via (at 119.38 99.06) (size 0.8) (drill 0.4) (layers "F.Cu" "B.Cu") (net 13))
 (segment (start 124.46 88.9) (end 119.38 93.98) (width 0.25) (layer "B.Cu") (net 13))
 (segment (start 119.38 93.98) (end 119.38 99.06) (width 0.25) (layer "B.Cu") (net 13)))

